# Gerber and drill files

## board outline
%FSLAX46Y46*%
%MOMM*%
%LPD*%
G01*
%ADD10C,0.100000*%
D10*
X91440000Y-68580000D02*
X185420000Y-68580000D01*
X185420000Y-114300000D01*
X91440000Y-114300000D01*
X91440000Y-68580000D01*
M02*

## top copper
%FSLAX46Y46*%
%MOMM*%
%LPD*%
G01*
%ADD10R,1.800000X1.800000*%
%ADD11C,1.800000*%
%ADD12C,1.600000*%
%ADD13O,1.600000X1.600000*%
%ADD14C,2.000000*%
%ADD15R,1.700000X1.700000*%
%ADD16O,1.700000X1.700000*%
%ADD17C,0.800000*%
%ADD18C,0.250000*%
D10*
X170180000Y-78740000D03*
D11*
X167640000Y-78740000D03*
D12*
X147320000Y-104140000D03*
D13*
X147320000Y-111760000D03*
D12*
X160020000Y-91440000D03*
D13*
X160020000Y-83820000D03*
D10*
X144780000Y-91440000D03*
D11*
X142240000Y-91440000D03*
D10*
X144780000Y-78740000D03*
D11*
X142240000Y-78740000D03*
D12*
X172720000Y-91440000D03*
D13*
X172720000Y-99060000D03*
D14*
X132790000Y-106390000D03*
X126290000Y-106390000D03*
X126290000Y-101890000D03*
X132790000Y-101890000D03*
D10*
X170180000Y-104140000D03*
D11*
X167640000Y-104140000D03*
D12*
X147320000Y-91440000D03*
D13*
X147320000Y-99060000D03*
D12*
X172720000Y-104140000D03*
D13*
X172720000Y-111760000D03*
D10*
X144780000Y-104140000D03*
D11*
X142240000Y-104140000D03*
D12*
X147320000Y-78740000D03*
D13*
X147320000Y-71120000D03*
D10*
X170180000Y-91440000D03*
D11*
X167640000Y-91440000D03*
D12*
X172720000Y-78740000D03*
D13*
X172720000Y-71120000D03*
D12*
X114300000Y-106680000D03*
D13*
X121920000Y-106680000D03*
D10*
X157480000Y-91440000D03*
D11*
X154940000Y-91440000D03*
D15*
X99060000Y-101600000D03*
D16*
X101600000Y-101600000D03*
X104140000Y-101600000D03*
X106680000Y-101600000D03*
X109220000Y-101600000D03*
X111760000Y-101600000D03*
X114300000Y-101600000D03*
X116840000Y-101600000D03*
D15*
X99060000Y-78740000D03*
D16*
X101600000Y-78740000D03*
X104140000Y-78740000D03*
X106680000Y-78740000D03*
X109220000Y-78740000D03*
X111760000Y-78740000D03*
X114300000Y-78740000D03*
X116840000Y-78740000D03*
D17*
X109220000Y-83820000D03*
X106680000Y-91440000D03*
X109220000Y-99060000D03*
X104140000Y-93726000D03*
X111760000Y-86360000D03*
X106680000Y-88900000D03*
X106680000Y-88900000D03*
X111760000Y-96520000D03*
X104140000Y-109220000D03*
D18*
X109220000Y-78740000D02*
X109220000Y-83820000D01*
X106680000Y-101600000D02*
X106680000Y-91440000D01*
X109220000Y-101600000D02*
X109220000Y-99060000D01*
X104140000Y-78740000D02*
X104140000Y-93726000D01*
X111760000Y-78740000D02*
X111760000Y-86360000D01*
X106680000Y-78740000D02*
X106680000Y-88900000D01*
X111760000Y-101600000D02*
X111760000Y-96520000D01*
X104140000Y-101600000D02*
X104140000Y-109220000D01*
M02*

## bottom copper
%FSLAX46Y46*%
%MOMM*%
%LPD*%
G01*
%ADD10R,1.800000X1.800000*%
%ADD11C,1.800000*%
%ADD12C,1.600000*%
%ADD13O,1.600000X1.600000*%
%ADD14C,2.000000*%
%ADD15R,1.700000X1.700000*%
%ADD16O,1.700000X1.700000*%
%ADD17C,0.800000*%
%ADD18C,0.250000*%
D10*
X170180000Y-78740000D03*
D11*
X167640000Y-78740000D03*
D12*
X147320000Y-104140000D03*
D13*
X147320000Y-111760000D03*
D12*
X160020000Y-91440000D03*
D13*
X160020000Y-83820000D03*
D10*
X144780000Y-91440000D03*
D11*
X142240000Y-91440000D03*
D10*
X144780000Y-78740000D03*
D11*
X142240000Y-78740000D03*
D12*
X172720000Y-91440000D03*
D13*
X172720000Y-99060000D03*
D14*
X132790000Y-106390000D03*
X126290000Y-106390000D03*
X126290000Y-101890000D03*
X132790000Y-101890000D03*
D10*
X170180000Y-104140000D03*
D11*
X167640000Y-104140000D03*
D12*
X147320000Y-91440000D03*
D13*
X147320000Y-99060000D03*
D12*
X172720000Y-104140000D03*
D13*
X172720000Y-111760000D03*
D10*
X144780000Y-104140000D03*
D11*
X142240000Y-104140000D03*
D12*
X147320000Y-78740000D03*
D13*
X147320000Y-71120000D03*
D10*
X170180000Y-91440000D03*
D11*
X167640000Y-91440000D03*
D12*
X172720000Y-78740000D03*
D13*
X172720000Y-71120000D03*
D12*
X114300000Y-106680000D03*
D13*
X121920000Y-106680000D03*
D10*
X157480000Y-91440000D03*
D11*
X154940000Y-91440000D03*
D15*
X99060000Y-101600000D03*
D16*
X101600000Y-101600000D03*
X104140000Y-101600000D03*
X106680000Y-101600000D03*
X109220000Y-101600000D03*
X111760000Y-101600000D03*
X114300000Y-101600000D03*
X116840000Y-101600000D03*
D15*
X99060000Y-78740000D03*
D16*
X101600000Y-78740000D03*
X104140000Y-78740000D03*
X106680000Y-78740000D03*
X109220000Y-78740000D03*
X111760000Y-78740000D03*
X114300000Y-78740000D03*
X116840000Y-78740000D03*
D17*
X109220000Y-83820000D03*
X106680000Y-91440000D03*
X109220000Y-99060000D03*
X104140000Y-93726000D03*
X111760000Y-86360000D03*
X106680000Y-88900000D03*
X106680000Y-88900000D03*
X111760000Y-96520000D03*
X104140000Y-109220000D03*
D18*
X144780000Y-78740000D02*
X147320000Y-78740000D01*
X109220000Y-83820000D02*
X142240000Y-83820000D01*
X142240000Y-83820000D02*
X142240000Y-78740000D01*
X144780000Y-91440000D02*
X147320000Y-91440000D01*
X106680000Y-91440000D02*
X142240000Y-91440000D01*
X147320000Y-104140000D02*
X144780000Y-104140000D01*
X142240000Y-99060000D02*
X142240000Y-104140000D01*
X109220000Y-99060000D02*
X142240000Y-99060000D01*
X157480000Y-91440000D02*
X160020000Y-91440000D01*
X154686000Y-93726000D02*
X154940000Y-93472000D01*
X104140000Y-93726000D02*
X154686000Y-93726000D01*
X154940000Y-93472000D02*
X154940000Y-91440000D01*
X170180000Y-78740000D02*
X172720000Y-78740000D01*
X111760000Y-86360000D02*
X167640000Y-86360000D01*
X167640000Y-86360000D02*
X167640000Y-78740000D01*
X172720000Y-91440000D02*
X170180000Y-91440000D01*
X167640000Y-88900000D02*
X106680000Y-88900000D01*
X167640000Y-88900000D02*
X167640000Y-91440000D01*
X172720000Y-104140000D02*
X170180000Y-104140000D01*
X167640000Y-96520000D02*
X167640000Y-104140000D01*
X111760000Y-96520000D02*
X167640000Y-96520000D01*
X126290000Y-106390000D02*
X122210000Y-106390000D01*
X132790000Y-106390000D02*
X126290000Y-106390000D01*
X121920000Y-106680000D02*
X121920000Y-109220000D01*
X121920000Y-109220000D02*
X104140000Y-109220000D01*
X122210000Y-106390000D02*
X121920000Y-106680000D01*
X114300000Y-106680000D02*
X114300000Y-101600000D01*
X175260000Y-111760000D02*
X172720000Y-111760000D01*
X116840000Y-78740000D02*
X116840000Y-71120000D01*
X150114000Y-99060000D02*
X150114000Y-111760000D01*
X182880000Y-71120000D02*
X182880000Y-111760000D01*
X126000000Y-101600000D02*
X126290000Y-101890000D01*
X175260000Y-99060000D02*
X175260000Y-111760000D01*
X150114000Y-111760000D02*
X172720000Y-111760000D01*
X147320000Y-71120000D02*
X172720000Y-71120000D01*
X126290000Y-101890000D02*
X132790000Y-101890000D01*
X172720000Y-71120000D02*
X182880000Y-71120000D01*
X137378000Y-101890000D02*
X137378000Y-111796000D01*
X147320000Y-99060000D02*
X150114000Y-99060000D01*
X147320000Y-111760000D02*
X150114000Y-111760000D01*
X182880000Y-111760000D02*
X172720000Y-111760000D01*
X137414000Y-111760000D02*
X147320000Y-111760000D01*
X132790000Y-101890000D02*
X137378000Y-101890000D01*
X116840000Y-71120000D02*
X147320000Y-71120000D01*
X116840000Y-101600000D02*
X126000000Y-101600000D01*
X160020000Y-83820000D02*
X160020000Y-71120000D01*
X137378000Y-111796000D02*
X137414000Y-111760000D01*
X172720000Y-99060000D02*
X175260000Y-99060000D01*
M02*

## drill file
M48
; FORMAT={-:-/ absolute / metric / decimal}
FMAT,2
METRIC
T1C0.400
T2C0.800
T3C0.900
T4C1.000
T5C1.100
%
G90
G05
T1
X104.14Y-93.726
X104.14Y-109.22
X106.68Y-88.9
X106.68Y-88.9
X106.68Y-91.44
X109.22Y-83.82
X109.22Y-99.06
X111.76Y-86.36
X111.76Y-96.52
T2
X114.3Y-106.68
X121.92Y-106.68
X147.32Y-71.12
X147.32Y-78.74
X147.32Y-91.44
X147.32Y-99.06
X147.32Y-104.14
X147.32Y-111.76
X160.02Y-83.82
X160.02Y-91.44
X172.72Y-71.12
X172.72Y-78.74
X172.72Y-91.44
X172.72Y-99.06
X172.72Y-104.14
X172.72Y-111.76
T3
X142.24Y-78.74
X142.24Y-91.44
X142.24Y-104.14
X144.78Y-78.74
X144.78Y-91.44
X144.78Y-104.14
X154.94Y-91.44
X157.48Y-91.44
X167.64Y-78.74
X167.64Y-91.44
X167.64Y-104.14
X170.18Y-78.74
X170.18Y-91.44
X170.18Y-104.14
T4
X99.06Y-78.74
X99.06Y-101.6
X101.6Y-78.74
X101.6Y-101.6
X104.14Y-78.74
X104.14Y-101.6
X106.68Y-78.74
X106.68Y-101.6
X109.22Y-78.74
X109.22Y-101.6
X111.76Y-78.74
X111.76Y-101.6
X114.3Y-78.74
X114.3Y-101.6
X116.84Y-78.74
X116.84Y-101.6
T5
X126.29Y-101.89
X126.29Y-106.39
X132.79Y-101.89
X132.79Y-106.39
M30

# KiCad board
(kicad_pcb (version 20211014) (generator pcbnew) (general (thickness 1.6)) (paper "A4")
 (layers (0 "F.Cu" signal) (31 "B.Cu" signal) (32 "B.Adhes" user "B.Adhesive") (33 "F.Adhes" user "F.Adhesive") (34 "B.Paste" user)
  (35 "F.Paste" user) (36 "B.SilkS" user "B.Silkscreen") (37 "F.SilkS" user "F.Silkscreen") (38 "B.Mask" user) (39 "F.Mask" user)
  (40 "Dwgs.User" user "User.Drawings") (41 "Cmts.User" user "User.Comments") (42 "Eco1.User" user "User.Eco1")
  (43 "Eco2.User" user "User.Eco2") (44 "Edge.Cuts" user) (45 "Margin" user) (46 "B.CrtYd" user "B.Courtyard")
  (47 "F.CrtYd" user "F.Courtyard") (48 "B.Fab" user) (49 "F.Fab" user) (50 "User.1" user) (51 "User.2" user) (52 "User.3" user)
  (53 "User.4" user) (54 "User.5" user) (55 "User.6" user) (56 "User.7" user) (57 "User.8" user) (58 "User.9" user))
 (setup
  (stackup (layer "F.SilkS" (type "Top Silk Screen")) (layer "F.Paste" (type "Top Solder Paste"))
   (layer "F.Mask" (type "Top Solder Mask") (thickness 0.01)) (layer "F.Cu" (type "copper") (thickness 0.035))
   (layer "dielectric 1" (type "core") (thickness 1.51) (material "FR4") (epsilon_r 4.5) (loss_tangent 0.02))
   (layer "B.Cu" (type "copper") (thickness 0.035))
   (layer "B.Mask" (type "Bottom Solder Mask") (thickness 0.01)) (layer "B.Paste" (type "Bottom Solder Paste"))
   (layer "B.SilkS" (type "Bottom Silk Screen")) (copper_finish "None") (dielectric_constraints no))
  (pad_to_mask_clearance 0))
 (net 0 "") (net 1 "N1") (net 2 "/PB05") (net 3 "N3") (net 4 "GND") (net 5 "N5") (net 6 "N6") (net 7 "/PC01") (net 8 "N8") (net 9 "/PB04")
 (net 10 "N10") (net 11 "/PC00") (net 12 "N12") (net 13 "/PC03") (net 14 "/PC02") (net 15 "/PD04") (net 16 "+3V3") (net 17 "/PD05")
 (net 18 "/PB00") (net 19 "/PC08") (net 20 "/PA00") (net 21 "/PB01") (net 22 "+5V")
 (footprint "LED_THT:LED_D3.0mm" (layer "F.Cu") (at 170.18 78.74 180)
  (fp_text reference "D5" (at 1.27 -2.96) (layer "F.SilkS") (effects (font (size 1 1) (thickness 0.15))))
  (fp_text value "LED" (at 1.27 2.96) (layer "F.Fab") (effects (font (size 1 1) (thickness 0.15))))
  (pad "1" thru_hole rect (at 0 0 180) (size 1.8 1.8) (drill 0.9) (layers *.Cu *.Mask) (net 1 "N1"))
  (pad "2" thru_hole circle (at 2.54 0 180) (size 1.8 1.8) (drill 0.9) (layers *.Cu *.Mask) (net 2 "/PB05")))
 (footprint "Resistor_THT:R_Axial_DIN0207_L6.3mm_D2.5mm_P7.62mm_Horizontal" (layer "F.Cu") (at 147.32 104.14 -90)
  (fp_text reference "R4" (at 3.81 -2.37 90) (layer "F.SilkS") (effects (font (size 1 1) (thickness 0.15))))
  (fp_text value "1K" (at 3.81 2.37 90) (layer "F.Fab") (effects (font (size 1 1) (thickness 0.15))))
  (pad "1" thru_hole circle (at 0 0 270) (size 1.6 1.6) (drill 0.8) (layers *.Cu *.Mask) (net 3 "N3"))
  (pad "2" thru_hole oval (at 7.62 0 270) (size 1.6 1.6) (drill 0.8) (layers *.Cu *.Mask) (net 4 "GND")))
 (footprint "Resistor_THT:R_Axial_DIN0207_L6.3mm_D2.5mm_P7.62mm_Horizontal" (layer "F.Cu") (at 160.02 91.44 90)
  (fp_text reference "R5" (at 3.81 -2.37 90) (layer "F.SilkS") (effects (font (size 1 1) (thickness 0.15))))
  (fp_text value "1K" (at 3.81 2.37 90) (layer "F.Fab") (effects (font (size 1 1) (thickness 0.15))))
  (pad "1" thru_hole circle (at 0 0 90) (size 1.6 1.6) (drill 0.8) (layers *.Cu *.Mask) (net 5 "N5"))
  (pad "2" thru_hole oval (at 7.62 0 90) (size 1.6 1.6) (drill 0.8) (layers *.Cu *.Mask) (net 4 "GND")))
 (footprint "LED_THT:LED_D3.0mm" (layer "F.Cu") (at 144.78 91.44 180)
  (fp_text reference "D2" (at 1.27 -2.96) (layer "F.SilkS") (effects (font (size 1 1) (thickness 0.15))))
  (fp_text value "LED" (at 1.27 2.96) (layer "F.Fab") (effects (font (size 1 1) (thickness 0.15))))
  (pad "1" thru_hole rect (at 0 0 180) (size 1.8 1.8) (drill 0.9) (layers *.Cu *.Mask) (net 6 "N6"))
  (pad "2" thru_hole circle (at 2.54 0 180) (size 1.8 1.8) (drill 0.9) (layers *.Cu *.Mask) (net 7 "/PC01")))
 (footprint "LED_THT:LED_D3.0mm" (layer "F.Cu") (at 144.78 78.74 180)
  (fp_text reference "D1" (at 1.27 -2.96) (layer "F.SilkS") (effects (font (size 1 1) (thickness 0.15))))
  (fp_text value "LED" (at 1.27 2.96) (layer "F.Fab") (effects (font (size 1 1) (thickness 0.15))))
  (pad "1" thru_hole rect (at 0 0 180) (size 1.8 1.8) (drill 0.9) (layers *.Cu *.Mask) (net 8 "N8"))
  (pad "2" thru_hole circle (at 2.54 0 180) (size 1.8 1.8) (drill 0.9) (layers *.Cu *.Mask) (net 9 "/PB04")))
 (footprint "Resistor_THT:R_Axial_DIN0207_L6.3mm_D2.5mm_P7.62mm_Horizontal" (layer "F.Cu") (at 172.72 91.44 -90)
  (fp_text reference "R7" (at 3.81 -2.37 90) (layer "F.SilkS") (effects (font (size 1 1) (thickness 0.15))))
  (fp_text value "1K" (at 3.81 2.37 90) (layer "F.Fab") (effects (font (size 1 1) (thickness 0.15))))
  (pad "1" thru_hole circle (at 0 0 270) (size 1.6 1.6) (drill 0.8) (layers *.Cu *.Mask) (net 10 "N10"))
  (pad "2" thru_hole oval (at 7.62 0 270) (size 1.6 1.6) (drill 0.8) (layers *.Cu *.Mask) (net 4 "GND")))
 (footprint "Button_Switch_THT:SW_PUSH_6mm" (layer "F.Cu") (at 132.79 106.39 180)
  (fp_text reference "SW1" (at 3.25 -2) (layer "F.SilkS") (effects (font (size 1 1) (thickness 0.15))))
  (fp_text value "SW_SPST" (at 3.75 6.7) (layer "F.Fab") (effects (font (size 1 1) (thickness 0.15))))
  (pad "1" thru_hole circle (at 0 0 270) (size 2 2) (drill 1.1) (layers *.Cu *.Mask) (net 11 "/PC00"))
  (pad "1" thru_hole circle (at 6.5 0 270) (size 2 2) (drill 1.1) (layers *.Cu *.Mask) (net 11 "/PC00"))
  (pad "2" thru_hole circle (at 6.5 4.5 270) (size 2 2) (drill 1.1) (layers *.Cu *.Mask) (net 4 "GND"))
  (pad "2" thru_hole circle (at 0 4.5 270) (size 2 2) (drill 1.1) (layers *.Cu *.Mask) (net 4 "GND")))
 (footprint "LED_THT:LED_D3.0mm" (layer "F.Cu") (at 170.18 104.14 180)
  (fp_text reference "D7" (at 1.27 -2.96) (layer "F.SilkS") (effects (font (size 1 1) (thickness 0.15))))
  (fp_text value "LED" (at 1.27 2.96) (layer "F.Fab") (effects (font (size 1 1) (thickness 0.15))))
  (pad "1" thru_hole rect (at 0 0 180) (size 1.8 1.8) (drill 0.9) (layers *.Cu *.Mask) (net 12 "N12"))
  (pad "2" thru_hole circle (at 2.54 0 180) (size 1.8 1.8) (drill 0.9) (layers *.Cu *.Mask) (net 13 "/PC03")))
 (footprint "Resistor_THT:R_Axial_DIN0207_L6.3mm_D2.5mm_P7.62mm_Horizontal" (layer "F.Cu") (at 147.32 91.44 -90)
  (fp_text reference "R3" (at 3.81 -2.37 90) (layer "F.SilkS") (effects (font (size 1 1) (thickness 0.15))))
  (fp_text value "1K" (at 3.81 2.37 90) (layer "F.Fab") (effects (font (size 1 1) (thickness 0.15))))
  (pad "1" thru_hole circle (at 0 0 270) (size 1.6 1.6) (drill 0.8) (layers *.Cu *.Mask) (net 6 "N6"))
  (pad "2" thru_hole oval (at 7.62 0 270) (size 1.6 1.6) (drill 0.8) (layers *.Cu *.Mask) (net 4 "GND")))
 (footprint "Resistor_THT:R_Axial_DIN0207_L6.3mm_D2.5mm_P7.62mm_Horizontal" (layer "F.Cu") (at 172.72 104.14 -90)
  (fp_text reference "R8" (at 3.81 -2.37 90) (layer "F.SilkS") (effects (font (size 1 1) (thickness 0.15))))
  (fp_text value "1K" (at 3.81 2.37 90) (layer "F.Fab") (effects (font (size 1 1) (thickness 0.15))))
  (pad "1" thru_hole circle (at 0 0 270) (size 1.6 1.6) (drill 0.8) (layers *.Cu *.Mask) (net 12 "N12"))
  (pad "2" thru_hole oval (at 7.62 0 270) (size 1.6 1.6) (drill 0.8) (layers *.Cu *.Mask) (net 4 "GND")))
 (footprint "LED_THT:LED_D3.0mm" (layer "F.Cu") (at 144.78 104.14 180)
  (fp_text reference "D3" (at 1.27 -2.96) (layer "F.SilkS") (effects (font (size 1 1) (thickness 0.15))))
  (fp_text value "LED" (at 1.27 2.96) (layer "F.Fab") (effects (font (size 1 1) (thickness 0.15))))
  (pad "1" thru_hole rect (at 0 0 180) (size 1.8 1.8) (drill 0.9) (layers *.Cu *.Mask) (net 3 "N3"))
  (pad "2" thru_hole circle (at 2.54 0 180) (size 1.8 1.8) (drill 0.9) (layers *.Cu *.Mask) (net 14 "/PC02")))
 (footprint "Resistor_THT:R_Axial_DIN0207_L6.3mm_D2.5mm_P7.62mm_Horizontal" (layer "F.Cu") (at 147.32 78.74 90)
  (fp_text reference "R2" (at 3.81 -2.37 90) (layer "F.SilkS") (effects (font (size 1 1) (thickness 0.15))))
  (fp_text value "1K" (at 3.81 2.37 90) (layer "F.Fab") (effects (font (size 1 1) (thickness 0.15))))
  (pad "1" thru_hole circle (at 0 0 90) (size 1.6 1.6) (drill 0.8) (layers *.Cu *.Mask) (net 8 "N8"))
  (pad "2" thru_hole oval (at 7.62 0 90) (size 1.6 1.6) (drill 0.8) (layers *.Cu *.Mask) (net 4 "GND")))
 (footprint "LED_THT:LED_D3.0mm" (layer "F.Cu") (at 170.18 91.44 180)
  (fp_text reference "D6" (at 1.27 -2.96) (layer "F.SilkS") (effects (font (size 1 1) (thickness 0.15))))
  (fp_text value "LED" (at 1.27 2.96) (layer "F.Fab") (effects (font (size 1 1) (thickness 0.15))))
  (pad "1" thru_hole rect (at 0 0 180) (size 1.8 1.8) (drill 0.9) (layers *.Cu *.Mask) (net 10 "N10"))
  (pad "2" thru_hole circle (at 2.54 0 180) (size 1.8 1.8) (drill 0.9) (layers *.Cu *.Mask) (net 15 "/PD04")))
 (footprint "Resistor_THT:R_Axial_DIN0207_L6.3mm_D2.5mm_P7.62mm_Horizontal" (layer "F.Cu") (at 172.72 78.74 90)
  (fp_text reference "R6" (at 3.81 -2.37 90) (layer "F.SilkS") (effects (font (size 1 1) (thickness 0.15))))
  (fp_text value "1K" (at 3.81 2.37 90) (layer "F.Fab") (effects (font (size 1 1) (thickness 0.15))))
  (pad "1" thru_hole circle (at 0 0 90) (size 1.6 1.6) (drill 0.8) (layers *.Cu *.Mask) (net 1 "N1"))
  (pad "2" thru_hole oval (at 7.62 0 90) (size 1.6 1.6) (drill 0.8) (layers *.Cu *.Mask) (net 4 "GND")))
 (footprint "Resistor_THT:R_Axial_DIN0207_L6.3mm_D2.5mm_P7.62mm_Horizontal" (layer "F.Cu") (at 114.3 106.68)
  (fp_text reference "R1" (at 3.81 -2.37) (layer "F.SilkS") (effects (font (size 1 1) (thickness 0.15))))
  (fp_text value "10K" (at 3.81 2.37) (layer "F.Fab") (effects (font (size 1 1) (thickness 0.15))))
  (pad "1" thru_hole circle (at 0 0) (size 1.6 1.6) (drill 0.8) (layers *.Cu *.Mask) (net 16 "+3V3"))
  (pad "2" thru_hole oval (at 7.62 0) (size 1.6 1.6) (drill 0.8) (layers *.Cu *.Mask) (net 11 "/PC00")))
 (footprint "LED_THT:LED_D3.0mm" (layer "F.Cu") (at 157.48 91.44 180)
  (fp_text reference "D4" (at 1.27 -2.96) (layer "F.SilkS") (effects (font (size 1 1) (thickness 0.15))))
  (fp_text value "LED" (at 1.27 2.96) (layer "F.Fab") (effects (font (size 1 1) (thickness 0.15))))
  (pad "1" thru_hole rect (at 0 0 180) (size 1.8 1.8) (drill 0.9) (layers *.Cu *.Mask) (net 5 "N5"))
  (pad "2" thru_hole circle (at 2.54 0 180) (size 1.8 1.8) (drill 0.9) (layers *.Cu *.Mask) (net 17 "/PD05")))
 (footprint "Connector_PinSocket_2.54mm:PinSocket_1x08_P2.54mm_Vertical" (layer "B.Cu") (at 99.06 101.6 -90)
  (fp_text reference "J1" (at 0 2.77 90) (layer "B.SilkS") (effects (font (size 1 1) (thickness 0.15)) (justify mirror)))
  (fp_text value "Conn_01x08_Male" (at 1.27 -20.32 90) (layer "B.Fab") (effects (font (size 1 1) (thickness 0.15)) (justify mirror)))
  (pad "1" thru_hole rect (at 0 0 270) (size 1.7 1.7) (drill 1) (layers *.Cu *.Mask) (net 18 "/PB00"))
  (pad "2" thru_hole oval (at 0 -2.54 270) (size 1.7 1.7) (drill 1) (layers *.Cu *.Mask) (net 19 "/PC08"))
  (pad "3" thru_hole oval (at 0 -5.08 270) (size 1.7 1.7) (drill 1) (layers *.Cu *.Mask) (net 11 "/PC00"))
  (pad "4" thru_hole oval (at 0 -7.62 270) (size 1.7 1.7) (drill 1) (layers *.Cu *.Mask) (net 7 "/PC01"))
  (pad "5" thru_hole oval (at 0 -10.16 270) (size 1.7 1.7) (drill 1) (layers *.Cu *.Mask) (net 14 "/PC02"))
  (pad "6" thru_hole oval (at 0 -12.7 270) (size 1.7 1.7) (drill 1) (layers *.Cu *.Mask) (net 13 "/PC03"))
  (pad "7" thru_hole oval (at 0 -15.24 270) (size 1.7 1.7) (drill 1) (layers *.Cu *.Mask) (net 16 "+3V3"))
  (pad "8" thru_hole oval (at 0 -17.78 270) (size 1.7 1.7) (drill 1) (layers *.Cu *.Mask) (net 4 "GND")))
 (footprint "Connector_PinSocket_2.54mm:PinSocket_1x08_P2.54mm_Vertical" (layer "B.Cu") (at 99.06 78.74 -90)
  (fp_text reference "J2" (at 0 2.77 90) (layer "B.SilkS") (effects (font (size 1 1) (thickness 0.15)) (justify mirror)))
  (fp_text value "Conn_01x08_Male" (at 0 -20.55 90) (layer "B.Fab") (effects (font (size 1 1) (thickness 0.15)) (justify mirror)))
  (pad "1" thru_hole rect (at 0 0 270) (size 1.7 1.7) (drill 1) (layers *.Cu *.Mask) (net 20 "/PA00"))
  (pad "2" thru_hole oval (at 0 -2.54 270) (size 1.7 1.7) (drill 1) (layers *.Cu *.Mask) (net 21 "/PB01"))
  (pad "3" thru_hole oval (at 0 -5.08 270) (size 1.7 1.7) (drill 1) (layers *.Cu *.Mask) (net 17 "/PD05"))
  (pad "4" thru_hole oval (at 0 -7.62 270) (size 1.7 1.7) (drill 1) (layers *.Cu *.Mask) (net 15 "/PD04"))
  (pad "5" thru_hole oval (at 0 -10.16 270) (size 1.7 1.7) (drill 1) (layers *.Cu *.Mask) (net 9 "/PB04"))
  (pad "6" thru_hole oval (at 0 -12.7 270) (size 1.7 1.7) (drill 1) (layers *.Cu *.Mask) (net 2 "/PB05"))
  (pad "7" thru_hole oval (at 0 -15.24 270) (size 1.7 1.7) (drill 1) (layers *.Cu *.Mask) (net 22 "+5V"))
  (pad "8" thru_hole oval (at 0 -17.78 270) (size 1.7 1.7) (drill 1) (layers *.Cu *.Mask) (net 4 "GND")))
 (gr_rect (start 91.44 68.58) (end 185.42 114.3) (layer "Edge.Cuts") (width 0.1) (fill none))
 (segment (start 144.78 78.74) (end 147.32 78.74) (width 0.25) (layer "B.Cu") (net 8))
 (segment (start 109.22 78.74) (end 109.22 83.82) (width 0.25) (layer "F.Cu") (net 9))
 (via (at 109.22 83.82) (size 0.8) (drill 0.4) (layers "F.Cu" "B.Cu") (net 9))
 (segment (start 109.22 83.82) (end 142.24 83.82) (width 0.25) (layer "B.Cu") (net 9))
 (segment (start 142.24 83.82) (end 142.24 78.74) (width 0.25) (layer "B.Cu") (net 9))
 (segment (start 144.78 91.44) (end 147.32 91.44) (width 0.25) (layer "B.Cu") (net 6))
 (segment (start 106.68 101.6) (end 106.68 91.44) (width 0.25) (layer "F.Cu") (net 7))
 (via (at 106.68 91.44) (size 0.8) (drill 0.4) (layers "F.Cu" "B.Cu") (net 7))
 (segment (start 106.68 91.44) (end 142.24 91.44) (width 0.25) (layer "B.Cu") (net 7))
 (segment (start 147.32 104.14) (end 144.78 104.14) (width 0.25) (layer "B.Cu") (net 3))
 (segment (start 109.22 101.6) (end 109.22 99.06) (width 0.25) (layer "F.Cu") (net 14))
 (via (at 109.22 99.06) (size 0.8) (drill 0.4) (layers "F.Cu" "B.Cu") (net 14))
 (segment (start 142.24 99.06) (end 142.24 104.14) (width 0.25) (layer "B.Cu") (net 14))
 (segment (start 109.22 99.06) (end 142.24 99.06) (width 0.25) (layer "B.Cu") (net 14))
 (segment (start 157.48 91.44) (end 160.02 91.44) (width 0.25) (layer "B.Cu") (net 5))
 (segment (start 104.14 78.74) (end 104.14 93.726) (width 0.25) (layer "F.Cu") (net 17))
 (via (at 104.14 93.726) (size 0.8) (drill 0.4) (layers "F.Cu" "B.Cu") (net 17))
 (segment (start 154.686 93.726) (end 154.94 93.472) (width 0.25) (layer "B.Cu") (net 17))
 (segment (start 104.14 93.726) (end 154.686 93.726) (width 0.25) (layer "B.Cu") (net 17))
 (segment (start 154.94 93.472) (end 154.94 91.44) (width 0.25) (layer "B.Cu") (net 17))
 (segment (start 170.18 78.74) (end 172.72 78.74) (width 0.25) (layer "B.Cu") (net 1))
 (segment (start 111.76 78.74) (end 111.76 86.36) (width 0.25) (layer "F.Cu") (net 2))
 (via (at 111.76 86.36) (size 0.8) (drill 0.4) (layers "F.Cu" "B.Cu") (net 2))
 (segment (start 111.76 86.36) (end 167.64 86.36) (width 0.25) (layer "B.Cu") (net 2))
 (segment (start 167.64 86.36) (end 167.64 78.74) (width 0.25) (layer "B.Cu") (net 2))
 (segment (start 172.72 91.44) (end 170.18 91.44) (width 0.25) (layer "B.Cu") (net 10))
 (segment (start 106.68 78.74) (end 106.68 88.9) (width 0.25) (layer "F.Cu") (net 15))
 (via (at 106.68 88.9) (size 0.8) (drill 0.4) (layers "F.Cu" "B.Cu") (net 15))
 (via (at 106.68 88.9) (size 0.8) (drill 0.4) (layers "F.Cu" "B.Cu") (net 15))
 (segment (start 167.64 88.9) (end 106.68 88.9) (width 0.25) (layer "B.Cu") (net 15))
 (segment (start 167.64 88.9) (end 167.64 91.44) (width 0.25) (layer "B.Cu") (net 15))
 (segment (start 172.72 104.14) (end 170.18 104.14) (width 0.25) (layer "B.Cu") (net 12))
 (segment (start 111.76 101.6) (end 111.76 96.52) (width 0.25) (layer "F.Cu") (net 13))
 (via (at 111.76 96.52) (size 0.8) (drill 0.4) (layers "F.Cu" "B.Cu") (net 13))
 (segment (start 167.64 96.52) (end 167.64 104.14) (width 0.25) (layer "B.Cu") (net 13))
 (segment (start 111.76 96.52) (end 167.64 96.52) (width 0.25) (layer "B.Cu") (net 13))
 (segment (start 104.14 101.6) (end 104.14 109.22) (width 0.25) (layer "F.Cu") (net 11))
 (via (at 104.14 109.22) (size 0.8) (drill 0.4) (layers "F.Cu" "B.Cu") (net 11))
 (segment (start 126.29 106.39) (end 122.21 106.39) (width 0.25) (layer "B.Cu") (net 11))
 (segment (start 132.79 106.39) (end 126.29 106.39) (width 0.25) (layer "B.Cu") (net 11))
 (segment (start 121.92 106.68) (end 121.92 109.22) (width 0.25) (layer "B.Cu") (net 11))
 (segment (start 121.92 109.22) (end 104.14 109.22) (width 0.25) (layer "B.Cu") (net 11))
 (segment (start 122.21 106.39) (end 121.92 106.68) (width 0.25) (layer "B.Cu") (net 11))
 (segment (start 114.3 106.68) (end 114.3 101.6) (width 0.25) (layer "B.Cu") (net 16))
 (segment (start 175.26 111.76) (end 172.72 111.76) (width 0.25) (layer "B.Cu") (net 4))
 (segment (start 116.84 78.74) (end 116.84 71.12) (width 0.25) (layer "B.Cu") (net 4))
 (segment (start 150.114 99.06) (end 150.114 111.76) (width 0.25) (layer "B.Cu") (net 4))
 (segment (start 182.88 71.12) (end 182.88 111.76) (width 0.25) (layer "B.Cu") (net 4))
 (segment (start 126 101.6) (end 126.29 101.89) (width 0.25) (layer "B.Cu") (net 4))
 (segment (start 175.26 99.06) (end 175.26 111.76) (width 0.25) (layer "B.Cu") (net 4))
 (segment (start 150.114 111.76) (end 172.72 111.76) (width 0.25) (layer "B.Cu") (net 4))
 (segment (start 147.32 71.12) (end 172.72 71.12) (width 0.25) (layer "B.Cu") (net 4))
 (segment (start 126.29 101.89) (end 132.79 101.89) (width 0.25) (layer "B.Cu") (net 4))
 (segment (start 172.72 71.12) (end 182.88 71.12) (width 0.25) (layer "B.Cu") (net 4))
 (segment (start 137.378 101.89) (end 137.378 111.796) (width 0.25) (layer "B.Cu") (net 4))
 (segment (start 147.32 99.06) (end 150.114 99.06) (width 0.25) (layer "B.Cu") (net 4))
 (segment (start 147.32 111.76) (end 150.114 111.76) (width 0.25) (layer "B.Cu") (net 4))
 (segment (start 182.88 111.76) (end 172.72 111.76) (width 0.25) (layer "B.Cu") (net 4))
 (segment (start 137.414 111.76) (end 147.32 111.76) (width 0.25) (layer "B.Cu") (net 4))
 (segment (start 132.79 101.89) (end 137.378 101.89) (width 0.25) (layer "B.Cu") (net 4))
 (segment (start 116.84 71.12) (end 147.32 71.12) (width 0.25) (layer "B.Cu") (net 4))
 (segment (start 116.84 101.6) (end 126 101.6) (width 0.25) (layer "B.Cu") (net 4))
 (segment (start 160.02 83.82) (end 160.02 71.12) (width 0.25) (layer "B.Cu") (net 4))
 (segment (start 137.378 111.796) (end 137.414 111.76) (width 0.25) (layer "B.Cu") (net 4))
 (segment (start 172.72 99.06) (end 175.26 99.06) (width 0.25) (layer "B.Cu") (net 4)))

